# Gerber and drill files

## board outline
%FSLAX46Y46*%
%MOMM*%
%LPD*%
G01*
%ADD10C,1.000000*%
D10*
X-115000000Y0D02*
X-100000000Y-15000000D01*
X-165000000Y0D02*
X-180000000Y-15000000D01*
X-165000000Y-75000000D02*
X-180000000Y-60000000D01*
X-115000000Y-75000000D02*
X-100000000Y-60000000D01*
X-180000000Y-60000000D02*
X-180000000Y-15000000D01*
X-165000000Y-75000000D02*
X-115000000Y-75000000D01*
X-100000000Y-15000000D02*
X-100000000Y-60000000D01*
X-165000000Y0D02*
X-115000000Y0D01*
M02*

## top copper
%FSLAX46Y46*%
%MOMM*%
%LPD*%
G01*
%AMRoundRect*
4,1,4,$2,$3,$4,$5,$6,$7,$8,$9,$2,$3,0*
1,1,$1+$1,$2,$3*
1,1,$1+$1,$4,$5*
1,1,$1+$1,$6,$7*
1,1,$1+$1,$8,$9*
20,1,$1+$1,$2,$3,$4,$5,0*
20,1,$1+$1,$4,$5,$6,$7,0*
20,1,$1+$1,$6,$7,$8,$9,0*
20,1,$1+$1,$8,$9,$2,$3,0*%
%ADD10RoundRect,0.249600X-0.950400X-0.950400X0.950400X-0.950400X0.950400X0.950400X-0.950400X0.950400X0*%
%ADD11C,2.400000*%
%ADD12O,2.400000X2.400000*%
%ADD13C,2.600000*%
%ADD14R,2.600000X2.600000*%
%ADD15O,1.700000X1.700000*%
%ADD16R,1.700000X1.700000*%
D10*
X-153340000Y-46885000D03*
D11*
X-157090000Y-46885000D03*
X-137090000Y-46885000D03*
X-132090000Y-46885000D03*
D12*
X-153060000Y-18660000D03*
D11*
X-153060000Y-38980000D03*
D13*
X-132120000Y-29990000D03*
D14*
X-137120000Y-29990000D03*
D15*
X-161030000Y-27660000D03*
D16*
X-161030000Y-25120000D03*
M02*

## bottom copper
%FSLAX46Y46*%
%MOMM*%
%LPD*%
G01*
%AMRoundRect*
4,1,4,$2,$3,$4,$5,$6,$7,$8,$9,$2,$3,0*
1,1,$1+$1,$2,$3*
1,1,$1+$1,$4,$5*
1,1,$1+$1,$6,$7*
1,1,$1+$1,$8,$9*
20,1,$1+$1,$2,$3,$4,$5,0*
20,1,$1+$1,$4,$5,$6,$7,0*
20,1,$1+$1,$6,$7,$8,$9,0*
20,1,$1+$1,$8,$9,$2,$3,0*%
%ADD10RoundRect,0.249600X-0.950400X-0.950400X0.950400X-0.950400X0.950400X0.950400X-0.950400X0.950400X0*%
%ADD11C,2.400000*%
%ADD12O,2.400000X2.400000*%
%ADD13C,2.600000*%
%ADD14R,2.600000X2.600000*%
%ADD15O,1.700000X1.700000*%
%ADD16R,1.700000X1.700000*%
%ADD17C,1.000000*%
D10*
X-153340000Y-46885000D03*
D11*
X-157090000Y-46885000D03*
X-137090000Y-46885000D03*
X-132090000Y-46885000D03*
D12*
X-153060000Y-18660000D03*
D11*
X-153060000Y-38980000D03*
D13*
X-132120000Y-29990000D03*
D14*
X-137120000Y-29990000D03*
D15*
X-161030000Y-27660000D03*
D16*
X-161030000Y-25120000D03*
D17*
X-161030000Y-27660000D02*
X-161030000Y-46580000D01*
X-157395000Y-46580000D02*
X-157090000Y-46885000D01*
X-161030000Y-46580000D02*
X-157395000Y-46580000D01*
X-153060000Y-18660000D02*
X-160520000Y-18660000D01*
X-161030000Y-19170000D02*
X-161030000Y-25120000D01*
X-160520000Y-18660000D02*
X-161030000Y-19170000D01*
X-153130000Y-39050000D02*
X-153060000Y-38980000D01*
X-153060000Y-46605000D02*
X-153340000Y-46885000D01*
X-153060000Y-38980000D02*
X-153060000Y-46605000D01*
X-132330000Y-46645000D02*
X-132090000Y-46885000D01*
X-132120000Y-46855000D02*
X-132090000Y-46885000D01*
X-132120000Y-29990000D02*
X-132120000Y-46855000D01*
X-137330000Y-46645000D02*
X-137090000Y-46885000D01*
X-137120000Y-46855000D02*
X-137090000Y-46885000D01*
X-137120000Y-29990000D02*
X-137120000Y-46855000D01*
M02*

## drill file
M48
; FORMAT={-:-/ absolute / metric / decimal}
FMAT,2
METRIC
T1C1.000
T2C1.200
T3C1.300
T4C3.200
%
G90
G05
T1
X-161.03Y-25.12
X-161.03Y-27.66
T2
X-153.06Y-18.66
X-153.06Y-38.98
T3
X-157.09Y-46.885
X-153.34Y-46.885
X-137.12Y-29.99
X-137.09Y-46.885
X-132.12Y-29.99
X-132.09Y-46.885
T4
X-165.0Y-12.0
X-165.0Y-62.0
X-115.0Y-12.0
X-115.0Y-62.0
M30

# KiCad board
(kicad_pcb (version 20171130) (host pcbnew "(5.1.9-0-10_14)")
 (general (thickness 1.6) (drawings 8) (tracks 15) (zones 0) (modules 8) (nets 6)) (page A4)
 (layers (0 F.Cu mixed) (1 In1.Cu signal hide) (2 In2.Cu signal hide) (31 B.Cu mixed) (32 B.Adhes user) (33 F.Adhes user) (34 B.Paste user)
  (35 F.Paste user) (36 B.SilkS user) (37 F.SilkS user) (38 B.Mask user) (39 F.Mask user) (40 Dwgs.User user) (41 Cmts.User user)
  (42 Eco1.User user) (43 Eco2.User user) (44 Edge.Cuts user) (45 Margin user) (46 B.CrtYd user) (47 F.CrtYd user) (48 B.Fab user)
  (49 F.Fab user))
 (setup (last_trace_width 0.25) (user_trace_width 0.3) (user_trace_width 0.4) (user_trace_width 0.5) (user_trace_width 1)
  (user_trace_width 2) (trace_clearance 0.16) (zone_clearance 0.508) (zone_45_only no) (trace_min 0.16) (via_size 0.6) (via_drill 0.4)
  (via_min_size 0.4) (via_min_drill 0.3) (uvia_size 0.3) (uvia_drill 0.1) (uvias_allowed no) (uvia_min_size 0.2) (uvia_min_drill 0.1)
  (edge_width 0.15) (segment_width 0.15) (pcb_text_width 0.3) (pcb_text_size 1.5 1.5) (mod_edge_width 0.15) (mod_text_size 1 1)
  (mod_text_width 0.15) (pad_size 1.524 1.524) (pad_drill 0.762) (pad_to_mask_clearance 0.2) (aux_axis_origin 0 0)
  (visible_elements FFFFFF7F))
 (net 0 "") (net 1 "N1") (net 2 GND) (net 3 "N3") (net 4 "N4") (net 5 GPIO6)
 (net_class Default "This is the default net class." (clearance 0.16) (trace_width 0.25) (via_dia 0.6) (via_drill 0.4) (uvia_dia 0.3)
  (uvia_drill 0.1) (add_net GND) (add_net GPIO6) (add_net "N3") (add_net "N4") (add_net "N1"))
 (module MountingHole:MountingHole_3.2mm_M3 (layer F.Cu) (at -165 62)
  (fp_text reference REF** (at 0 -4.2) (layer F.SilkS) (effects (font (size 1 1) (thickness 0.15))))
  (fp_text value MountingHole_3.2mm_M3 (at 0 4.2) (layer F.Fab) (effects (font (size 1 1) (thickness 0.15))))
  (pad 1 np_thru_hole circle (at 0 0) (size 3.2 3.2) (drill 3.2) (layers *.Cu *.Mask)))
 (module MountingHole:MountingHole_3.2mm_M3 (layer F.Cu) (at -115 62)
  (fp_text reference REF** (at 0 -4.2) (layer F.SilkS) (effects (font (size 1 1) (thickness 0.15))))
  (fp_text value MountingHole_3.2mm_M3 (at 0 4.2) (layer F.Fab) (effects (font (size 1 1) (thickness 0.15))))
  (pad 1 np_thru_hole circle (at 0 0) (size 3.2 3.2) (drill 3.2) (layers *.Cu *.Mask)))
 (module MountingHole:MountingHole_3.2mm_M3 (layer F.Cu) (at -115 12)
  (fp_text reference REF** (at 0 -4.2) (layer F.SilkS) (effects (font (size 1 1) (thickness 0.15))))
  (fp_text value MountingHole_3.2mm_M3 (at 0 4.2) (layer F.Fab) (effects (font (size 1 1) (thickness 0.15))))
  (pad 1 np_thru_hole circle (at 0 0) (size 3.2 3.2) (drill 3.2) (layers *.Cu *.Mask)))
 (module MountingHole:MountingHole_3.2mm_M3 (layer F.Cu) (at -165 12)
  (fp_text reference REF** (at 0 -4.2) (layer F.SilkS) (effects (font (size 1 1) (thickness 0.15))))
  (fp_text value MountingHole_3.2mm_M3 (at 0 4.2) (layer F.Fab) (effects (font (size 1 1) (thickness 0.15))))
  (pad 1 np_thru_hole circle (at 0 0) (size 3.2 3.2) (drill 3.2) (layers *.Cu *.Mask)))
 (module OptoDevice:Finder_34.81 (layer F.Cu) (at -153.34 46.885)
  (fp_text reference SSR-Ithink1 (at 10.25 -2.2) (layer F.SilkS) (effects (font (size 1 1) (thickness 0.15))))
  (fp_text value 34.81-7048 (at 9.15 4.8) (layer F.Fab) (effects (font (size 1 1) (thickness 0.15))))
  (pad A1 thru_hole roundrect (at 0 0) (size 2.4 2.4) (drill 1.3) (layers *.Cu *.Mask) (roundrect_rratio 0.104) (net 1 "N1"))
  (pad A2 thru_hole circle (at -3.75 0) (size 2.4 2.4) (drill 1.3) (layers *.Cu *.Mask) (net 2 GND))
  (pad 11 thru_hole circle (at 16.25 0) (size 2.4 2.4) (drill 1.3) (layers *.Cu *.Mask) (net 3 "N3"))
  (pad 14 thru_hole circle (at 21.25 0) (size 2.4 2.4) (drill 1.3) (layers *.Cu *.Mask) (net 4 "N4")))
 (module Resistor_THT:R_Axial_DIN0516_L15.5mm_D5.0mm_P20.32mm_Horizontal (layer F.Cu) (at -153.06 38.98 90)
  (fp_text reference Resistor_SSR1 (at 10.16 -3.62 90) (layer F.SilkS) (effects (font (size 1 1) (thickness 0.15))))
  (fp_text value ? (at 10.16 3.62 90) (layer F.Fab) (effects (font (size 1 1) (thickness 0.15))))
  (pad 2 thru_hole oval (at 20.32 0 90) (size 2.4 2.4) (drill 1.2) (layers *.Cu *.Mask) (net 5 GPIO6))
  (pad 1 thru_hole circle (at 0 0 90) (size 2.4 2.4) (drill 1.2) (layers *.Cu *.Mask) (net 1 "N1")))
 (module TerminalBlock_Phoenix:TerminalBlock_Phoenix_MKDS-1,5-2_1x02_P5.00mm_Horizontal (layer F.Cu) (at -137.12 29.99)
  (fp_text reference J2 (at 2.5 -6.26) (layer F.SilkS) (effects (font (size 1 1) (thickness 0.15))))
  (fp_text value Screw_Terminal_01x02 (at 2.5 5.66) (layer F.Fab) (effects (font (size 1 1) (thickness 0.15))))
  (pad 2 thru_hole circle (at 5 0) (size 2.6 2.6) (drill 1.3) (layers *.Cu *.Mask) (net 4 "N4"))
  (pad 1 thru_hole rect (at 0 0) (size 2.6 2.6) (drill 1.3) (layers *.Cu *.Mask) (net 3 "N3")))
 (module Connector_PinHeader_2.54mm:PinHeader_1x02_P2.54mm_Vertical (layer F.Cu) (at -161.03 25.12)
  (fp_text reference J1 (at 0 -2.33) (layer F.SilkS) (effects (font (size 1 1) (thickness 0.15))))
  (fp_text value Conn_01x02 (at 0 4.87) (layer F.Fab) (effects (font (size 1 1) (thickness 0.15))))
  (pad 2 thru_hole oval (at 0 2.54) (size 1.7 1.7) (drill 1) (layers *.Cu *.Mask) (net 2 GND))
  (pad 1 thru_hole rect (at 0 0) (size 1.7 1.7) (drill 1) (layers *.Cu *.Mask) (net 5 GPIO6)))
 (gr_line (start -115 0) (end -100 15) (layer Edge.Cuts) (width 1))
 (gr_line (start -165 0) (end -180 15) (layer Edge.Cuts) (width 1))
 (gr_line (start -165 75) (end -180 60) (layer Edge.Cuts) (width 1))
 (gr_line (start -115 75) (end -100 60) (layer Edge.Cuts) (width 1))
 (gr_line (start -180 60) (end -180 15) (layer Edge.Cuts) (width 1))
 (gr_line (start -165 75) (end -115 75) (layer Edge.Cuts) (width 1))
 (gr_line (start -100 15) (end -100 60) (layer Edge.Cuts) (width 1))
 (gr_line (start -165 0) (end -115 0) (layer Edge.Cuts) (width 1))
 (segment (start -161.03 27.66) (end -161.03 46.58) (width 1) (layer B.Cu) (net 2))
 (segment (start -157.395 46.58) (end -157.09 46.885) (width 1) (layer B.Cu) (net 2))
 (segment (start -161.03 46.58) (end -157.395 46.58) (width 1) (layer B.Cu) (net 2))
 (segment (start -153.06 18.66) (end -160.52 18.66) (width 1) (layer B.Cu) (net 5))
 (segment (start -161.03 19.17) (end -161.03 25.12) (width 1) (layer B.Cu) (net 5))
 (segment (start -160.52 18.66) (end -161.03 19.17) (width 1) (layer B.Cu) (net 5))
 (segment (start -153.13 39.05) (end -153.06 38.98) (width 1) (layer B.Cu) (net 1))
 (segment (start -153.06 46.605) (end -153.34 46.885) (width 1) (layer B.Cu) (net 1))
 (segment (start -153.06 38.98) (end -153.06 46.605) (width 1) (layer B.Cu) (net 1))
 (segment (start -132.33 46.645) (end -132.09 46.885) (width 1) (layer B.Cu) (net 4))
 (segment (start -132.12 46.855) (end -132.09 46.885) (width 1) (layer B.Cu) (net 4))
 (segment (start -132.12 29.99) (end -132.12 46.855) (width 1) (layer B.Cu) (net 4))
 (segment (start -137.33 46.645) (end -137.09 46.885) (width 1) (layer B.Cu) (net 3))
 (segment (start -137.12 46.855) (end -137.09 46.885) (width 1) (layer B.Cu) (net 3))
 (segment (start -137.12 29.99) (end -137.12 46.855) (width 1) (layer B.Cu) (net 3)))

